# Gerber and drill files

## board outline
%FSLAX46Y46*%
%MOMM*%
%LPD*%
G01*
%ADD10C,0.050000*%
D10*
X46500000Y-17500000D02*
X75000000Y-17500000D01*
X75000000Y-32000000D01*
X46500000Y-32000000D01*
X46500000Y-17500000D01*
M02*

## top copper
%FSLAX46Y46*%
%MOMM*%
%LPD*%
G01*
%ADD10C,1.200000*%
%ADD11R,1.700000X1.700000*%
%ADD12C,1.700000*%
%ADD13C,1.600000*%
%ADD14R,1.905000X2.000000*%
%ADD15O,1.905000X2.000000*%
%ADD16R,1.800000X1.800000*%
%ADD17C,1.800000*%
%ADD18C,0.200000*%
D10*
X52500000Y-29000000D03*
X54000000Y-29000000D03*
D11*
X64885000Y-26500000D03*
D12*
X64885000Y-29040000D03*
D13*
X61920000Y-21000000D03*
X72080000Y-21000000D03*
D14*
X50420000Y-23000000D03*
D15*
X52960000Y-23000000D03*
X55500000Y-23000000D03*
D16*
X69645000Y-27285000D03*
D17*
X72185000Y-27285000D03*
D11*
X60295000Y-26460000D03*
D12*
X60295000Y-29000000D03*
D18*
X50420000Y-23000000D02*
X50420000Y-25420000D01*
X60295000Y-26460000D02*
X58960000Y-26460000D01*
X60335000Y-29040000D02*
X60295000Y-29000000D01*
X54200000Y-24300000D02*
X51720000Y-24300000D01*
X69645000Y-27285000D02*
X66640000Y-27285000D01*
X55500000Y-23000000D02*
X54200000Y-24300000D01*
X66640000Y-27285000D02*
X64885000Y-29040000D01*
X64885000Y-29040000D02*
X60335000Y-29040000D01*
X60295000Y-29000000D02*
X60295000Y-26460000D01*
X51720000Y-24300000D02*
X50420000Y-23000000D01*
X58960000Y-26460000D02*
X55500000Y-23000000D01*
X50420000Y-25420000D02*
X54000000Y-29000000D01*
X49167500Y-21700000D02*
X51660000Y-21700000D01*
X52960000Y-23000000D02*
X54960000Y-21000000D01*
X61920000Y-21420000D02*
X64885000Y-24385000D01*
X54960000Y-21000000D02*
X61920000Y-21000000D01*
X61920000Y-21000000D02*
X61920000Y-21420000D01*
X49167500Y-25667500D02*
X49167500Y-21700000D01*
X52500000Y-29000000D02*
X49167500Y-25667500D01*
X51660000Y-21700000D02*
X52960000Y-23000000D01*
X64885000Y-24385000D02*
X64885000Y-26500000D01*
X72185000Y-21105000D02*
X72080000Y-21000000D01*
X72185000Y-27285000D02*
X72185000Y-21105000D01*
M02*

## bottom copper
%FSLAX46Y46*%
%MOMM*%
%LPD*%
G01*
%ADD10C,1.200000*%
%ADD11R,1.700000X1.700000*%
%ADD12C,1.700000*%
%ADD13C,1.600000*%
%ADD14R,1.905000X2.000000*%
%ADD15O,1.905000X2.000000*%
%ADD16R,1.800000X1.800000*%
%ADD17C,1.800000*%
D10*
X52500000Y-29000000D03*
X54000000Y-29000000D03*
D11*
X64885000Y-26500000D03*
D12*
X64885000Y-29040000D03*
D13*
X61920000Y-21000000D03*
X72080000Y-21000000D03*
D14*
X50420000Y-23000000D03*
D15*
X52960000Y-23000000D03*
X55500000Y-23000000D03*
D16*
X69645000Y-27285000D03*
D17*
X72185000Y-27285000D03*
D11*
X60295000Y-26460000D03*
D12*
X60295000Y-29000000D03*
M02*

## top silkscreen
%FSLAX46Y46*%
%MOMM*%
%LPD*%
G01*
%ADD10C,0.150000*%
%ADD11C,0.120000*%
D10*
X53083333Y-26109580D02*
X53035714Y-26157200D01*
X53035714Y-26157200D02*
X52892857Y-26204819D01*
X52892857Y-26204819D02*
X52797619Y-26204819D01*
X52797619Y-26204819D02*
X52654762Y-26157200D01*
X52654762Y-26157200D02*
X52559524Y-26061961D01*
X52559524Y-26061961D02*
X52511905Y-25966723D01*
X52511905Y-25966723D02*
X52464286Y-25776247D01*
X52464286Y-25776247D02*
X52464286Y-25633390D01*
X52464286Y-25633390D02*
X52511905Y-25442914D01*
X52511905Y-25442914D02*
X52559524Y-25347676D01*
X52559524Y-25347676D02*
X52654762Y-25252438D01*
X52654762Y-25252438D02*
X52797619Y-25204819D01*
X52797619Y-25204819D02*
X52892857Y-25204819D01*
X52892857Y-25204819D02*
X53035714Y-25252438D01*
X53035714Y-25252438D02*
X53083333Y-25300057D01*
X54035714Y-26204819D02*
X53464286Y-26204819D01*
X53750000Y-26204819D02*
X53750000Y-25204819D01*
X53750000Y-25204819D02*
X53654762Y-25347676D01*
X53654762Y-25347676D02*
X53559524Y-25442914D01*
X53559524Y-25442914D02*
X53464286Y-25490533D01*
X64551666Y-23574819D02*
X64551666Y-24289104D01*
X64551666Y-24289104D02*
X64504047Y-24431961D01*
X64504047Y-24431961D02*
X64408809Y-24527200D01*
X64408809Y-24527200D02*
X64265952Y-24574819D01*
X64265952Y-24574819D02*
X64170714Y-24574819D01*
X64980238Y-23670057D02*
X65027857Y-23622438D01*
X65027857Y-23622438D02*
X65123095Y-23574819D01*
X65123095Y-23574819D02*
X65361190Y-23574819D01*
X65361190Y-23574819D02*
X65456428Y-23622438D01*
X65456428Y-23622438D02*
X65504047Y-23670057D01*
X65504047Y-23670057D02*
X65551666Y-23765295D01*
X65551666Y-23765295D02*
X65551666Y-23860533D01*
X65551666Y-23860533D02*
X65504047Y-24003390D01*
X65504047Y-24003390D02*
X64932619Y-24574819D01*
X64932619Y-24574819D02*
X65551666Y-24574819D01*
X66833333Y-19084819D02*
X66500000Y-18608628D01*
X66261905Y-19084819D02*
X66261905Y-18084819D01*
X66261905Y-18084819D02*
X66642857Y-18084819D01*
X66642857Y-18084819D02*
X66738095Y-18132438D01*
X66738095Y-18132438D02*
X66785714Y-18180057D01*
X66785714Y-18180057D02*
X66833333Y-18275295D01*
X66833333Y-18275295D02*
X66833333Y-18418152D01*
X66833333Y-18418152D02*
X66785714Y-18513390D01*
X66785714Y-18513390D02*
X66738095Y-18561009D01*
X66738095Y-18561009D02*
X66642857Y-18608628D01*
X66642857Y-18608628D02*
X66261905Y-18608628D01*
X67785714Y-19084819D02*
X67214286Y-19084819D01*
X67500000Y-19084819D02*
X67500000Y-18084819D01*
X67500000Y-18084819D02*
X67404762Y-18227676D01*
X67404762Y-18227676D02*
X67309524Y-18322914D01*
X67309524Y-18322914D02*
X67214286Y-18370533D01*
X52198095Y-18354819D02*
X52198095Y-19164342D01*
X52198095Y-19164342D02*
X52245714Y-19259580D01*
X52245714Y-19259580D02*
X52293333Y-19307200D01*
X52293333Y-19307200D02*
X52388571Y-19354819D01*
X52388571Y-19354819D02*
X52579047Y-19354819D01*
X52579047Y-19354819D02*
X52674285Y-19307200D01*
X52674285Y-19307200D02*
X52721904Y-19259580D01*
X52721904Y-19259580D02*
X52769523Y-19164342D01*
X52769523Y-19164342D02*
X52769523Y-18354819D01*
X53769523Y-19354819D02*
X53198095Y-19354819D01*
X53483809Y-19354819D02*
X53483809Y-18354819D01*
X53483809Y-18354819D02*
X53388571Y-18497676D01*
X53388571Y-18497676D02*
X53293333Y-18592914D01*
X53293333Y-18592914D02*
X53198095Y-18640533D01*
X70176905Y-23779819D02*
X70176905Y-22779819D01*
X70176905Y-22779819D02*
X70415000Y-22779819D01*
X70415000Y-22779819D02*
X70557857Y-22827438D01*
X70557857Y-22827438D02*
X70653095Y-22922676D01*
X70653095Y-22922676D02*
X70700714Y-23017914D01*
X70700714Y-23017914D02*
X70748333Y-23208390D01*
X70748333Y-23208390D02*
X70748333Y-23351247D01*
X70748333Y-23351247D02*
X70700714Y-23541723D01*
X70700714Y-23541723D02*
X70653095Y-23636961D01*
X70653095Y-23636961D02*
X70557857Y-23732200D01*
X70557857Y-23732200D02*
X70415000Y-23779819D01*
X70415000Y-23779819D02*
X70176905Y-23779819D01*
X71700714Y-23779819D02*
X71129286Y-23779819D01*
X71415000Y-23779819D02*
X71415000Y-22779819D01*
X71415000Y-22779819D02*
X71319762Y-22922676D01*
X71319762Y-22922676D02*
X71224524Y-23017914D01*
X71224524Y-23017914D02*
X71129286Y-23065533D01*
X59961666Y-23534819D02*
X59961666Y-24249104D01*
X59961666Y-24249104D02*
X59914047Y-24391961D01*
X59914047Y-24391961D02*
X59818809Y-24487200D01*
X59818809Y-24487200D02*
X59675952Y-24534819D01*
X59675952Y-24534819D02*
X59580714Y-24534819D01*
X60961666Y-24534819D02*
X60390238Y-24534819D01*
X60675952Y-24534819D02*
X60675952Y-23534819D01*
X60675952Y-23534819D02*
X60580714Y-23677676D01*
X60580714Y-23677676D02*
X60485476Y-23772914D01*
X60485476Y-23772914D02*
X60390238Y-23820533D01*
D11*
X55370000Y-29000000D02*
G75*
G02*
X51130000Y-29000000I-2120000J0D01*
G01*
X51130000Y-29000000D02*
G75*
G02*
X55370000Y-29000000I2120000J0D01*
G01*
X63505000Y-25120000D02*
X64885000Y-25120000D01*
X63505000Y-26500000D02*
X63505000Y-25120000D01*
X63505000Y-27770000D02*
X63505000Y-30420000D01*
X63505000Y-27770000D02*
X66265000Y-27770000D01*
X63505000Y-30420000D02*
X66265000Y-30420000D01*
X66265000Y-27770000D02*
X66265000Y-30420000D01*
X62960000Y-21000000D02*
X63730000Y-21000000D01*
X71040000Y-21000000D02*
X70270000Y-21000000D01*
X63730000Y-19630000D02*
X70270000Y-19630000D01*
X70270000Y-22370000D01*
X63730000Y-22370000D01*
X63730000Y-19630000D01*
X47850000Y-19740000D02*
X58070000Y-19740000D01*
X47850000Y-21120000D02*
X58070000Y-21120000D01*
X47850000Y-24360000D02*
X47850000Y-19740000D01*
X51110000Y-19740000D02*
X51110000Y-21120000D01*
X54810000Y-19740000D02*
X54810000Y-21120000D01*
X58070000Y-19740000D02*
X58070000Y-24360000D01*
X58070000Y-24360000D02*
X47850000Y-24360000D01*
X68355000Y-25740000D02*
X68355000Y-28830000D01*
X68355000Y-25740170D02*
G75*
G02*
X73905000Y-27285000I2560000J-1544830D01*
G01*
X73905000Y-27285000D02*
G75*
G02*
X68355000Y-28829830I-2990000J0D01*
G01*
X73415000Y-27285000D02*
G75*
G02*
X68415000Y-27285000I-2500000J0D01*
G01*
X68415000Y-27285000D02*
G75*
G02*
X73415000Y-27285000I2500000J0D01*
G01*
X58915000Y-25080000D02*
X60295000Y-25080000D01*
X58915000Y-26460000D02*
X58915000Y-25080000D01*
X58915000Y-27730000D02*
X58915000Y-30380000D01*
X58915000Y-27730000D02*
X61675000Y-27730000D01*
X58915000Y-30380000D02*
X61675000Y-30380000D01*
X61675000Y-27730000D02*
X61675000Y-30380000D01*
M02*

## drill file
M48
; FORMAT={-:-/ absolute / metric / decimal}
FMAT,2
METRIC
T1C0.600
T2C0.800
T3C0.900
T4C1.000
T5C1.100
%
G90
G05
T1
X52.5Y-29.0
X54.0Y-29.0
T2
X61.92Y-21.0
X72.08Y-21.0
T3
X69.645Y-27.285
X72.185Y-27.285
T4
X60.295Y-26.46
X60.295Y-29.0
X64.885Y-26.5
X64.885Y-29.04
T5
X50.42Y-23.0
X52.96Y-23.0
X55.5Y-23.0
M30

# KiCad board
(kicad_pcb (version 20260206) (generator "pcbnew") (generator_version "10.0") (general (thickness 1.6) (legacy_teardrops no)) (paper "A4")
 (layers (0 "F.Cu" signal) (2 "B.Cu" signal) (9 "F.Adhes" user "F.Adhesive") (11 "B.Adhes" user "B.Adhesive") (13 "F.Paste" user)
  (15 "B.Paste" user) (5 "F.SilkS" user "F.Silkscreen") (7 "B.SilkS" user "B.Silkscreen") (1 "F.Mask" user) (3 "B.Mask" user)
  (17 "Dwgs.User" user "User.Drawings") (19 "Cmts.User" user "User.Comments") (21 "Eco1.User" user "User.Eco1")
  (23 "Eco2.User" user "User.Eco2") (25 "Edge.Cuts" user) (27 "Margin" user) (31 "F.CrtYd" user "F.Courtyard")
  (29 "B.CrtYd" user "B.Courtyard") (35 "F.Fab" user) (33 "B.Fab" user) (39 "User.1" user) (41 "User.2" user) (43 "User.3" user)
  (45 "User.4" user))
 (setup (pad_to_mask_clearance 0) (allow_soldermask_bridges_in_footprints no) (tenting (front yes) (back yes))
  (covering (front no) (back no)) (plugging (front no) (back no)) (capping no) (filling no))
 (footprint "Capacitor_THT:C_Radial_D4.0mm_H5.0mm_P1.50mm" (layer "F.Cu") (at 52.5 29)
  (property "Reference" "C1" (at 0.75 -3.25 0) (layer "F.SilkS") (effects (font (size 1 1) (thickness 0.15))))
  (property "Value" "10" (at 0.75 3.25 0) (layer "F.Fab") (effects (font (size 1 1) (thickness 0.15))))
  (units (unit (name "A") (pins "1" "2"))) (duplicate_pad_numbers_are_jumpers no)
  (fp_circle (center 0.75 0) (end 2.87 0) (stroke (width 0.12) (type solid)) (fill no) (layer "F.SilkS"))
  (pad "1" thru_hole circle (at 0 0) (size 1.2 1.2) (drill 0.6) (layers "*.Cu" "*.Mask") (remove_unused_layers no) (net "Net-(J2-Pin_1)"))
  (pad "2" thru_hole circle (at 1.5 0) (size 1.2 1.2) (drill 0.6) (layers "*.Cu" "*.Mask") (remove_unused_layers no) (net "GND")))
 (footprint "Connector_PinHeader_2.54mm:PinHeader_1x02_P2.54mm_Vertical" (layer "F.Cu") (at 64.885 26.5)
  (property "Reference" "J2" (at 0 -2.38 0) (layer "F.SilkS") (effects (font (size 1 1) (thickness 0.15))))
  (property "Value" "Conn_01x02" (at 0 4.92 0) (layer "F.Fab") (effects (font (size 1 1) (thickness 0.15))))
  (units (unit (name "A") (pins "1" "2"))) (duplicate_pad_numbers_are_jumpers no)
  (fp_line (start -1.38 -1.38) (end 0 -1.38) (stroke (width 0.12) (type solid)) (layer "F.SilkS"))
  (fp_line (start -1.38 0) (end -1.38 -1.38) (stroke (width 0.12) (type solid)) (layer "F.SilkS"))
  (fp_line (start -1.38 1.27) (end -1.38 3.92) (stroke (width 0.12) (type solid)) (layer "F.SilkS"))
  (fp_line (start -1.38 1.27) (end 1.38 1.27) (stroke (width 0.12) (type solid)) (layer "F.SilkS"))
  (fp_line (start -1.38 3.92) (end 1.38 3.92) (stroke (width 0.12) (type solid)) (layer "F.SilkS"))
  (fp_line (start 1.38 1.27) (end 1.38 3.92) (stroke (width 0.12) (type solid)) (layer "F.SilkS"))
  (pad "1" thru_hole rect (at 0 0) (size 1.7 1.7) (drill 1) (layers "*.Cu" "*.Mask") (remove_unused_layers no) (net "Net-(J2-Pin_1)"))
  (pad "2" thru_hole circle (at 0 2.54) (size 1.7 1.7) (drill 1) (layers "*.Cu" "*.Mask") (remove_unused_layers no) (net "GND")))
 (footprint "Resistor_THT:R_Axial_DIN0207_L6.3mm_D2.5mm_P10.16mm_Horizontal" (layer "F.Cu") (at 61.92 21)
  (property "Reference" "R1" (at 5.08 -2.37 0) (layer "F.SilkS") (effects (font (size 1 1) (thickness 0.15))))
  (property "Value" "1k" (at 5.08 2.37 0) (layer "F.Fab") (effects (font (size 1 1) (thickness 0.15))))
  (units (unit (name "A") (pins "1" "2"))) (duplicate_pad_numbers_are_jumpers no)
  (fp_line (start 1.04 0) (end 1.81 0) (stroke (width 0.12) (type solid)) (layer "F.SilkS"))
  (fp_line (start 9.12 0) (end 8.35 0) (stroke (width 0.12) (type solid)) (layer "F.SilkS"))
  (fp_rect (start 1.81 -1.37) (end 8.35 1.37) (stroke (width 0.12) (type solid)) (fill no) (layer "F.SilkS"))
  (pad "1" thru_hole circle (at 0 0) (size 1.6 1.6) (drill 0.8) (layers "*.Cu" "*.Mask") (remove_unused_layers no) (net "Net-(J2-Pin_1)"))
  (pad "2" thru_hole circle (at 10.16 0) (size 1.6 1.6) (drill 0.8) (layers "*.Cu" "*.Mask") (remove_unused_layers no) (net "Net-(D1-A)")))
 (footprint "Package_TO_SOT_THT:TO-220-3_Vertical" (layer "F.Cu") (at 50.42 23)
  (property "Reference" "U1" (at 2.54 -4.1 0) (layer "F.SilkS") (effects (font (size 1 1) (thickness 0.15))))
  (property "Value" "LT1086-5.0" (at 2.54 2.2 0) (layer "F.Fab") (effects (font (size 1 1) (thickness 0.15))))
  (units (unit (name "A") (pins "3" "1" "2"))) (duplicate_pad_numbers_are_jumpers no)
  (fp_line (start -2.57 -3.26) (end 7.65 -3.26) (stroke (width 0.12) (type solid)) (layer "F.SilkS"))
  (fp_line (start -2.57 -1.88) (end 7.65 -1.88) (stroke (width 0.12) (type solid)) (layer "F.SilkS"))
  (fp_line (start -2.57 1.36) (end -2.57 -3.26) (stroke (width 0.12) (type solid)) (layer "F.SilkS"))
  (fp_line (start 0.69 -3.26) (end 0.69 -1.88) (stroke (width 0.12) (type solid)) (layer "F.SilkS"))
  (fp_line (start 4.39 -3.26) (end 4.39 -1.88) (stroke (width 0.12) (type solid)) (layer "F.SilkS"))
  (fp_line (start 7.65 -3.26) (end 7.65 1.36) (stroke (width 0.12) (type solid)) (layer "F.SilkS"))
  (fp_line (start 7.65 1.36) (end -2.57 1.36) (stroke (width 0.12) (type solid)) (layer "F.SilkS"))
  (pad "1" thru_hole rect (at 0 0) (size 1.905 2) (drill 1.1) (layers "*.Cu" "*.Mask") (remove_unused_layers no) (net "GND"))
  (pad "2" thru_hole oval (at 2.54 0) (size 1.905 2) (drill 1.1) (layers "*.Cu" "*.Mask") (remove_unused_layers no) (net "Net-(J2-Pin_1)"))
  (pad "3" thru_hole oval (at 5.08 0) (size 1.905 2) (drill 1.1) (layers "*.Cu" "*.Mask") (remove_unused_layers no) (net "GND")))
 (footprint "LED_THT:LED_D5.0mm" (layer "F.Cu") (at 69.645 27.285)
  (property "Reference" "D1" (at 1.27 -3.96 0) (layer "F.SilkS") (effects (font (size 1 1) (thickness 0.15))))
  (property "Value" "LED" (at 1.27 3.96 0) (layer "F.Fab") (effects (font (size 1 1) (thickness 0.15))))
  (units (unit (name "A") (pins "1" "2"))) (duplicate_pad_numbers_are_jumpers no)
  (fp_line (start -1.29 -1.545) (end -1.29 1.545) (stroke (width 0.12) (type solid)) (layer "F.SilkS"))
  (fp_arc (start -1.29 -1.54483) (mid 2.071779 -2.880495) (end 4.26 0) (stroke (width 0.12) (type solid)) (layer "F.SilkS"))
  (fp_arc (start 4.26 0) (mid 2.071779 2.880495) (end -1.29 1.54483) (stroke (width 0.12) (type solid)) (layer "F.SilkS"))
  (fp_circle (center 1.27 0) (end 3.77 0) (stroke (width 0.12) (type solid)) (fill no) (layer "F.SilkS"))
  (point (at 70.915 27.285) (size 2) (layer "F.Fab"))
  (pad "1" thru_hole rect (at 0 0) (size 1.8 1.8) (drill 0.9) (layers "*.Cu" "*.Mask") (remove_unused_layers no) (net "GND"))
  (pad "2" thru_hole circle (at 2.54 0) (size 1.8 1.8) (drill 0.9) (layers "*.Cu" "*.Mask") (remove_unused_layers no) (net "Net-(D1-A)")))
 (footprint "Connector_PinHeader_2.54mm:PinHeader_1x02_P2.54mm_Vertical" (layer "F.Cu") (at 60.295 26.46)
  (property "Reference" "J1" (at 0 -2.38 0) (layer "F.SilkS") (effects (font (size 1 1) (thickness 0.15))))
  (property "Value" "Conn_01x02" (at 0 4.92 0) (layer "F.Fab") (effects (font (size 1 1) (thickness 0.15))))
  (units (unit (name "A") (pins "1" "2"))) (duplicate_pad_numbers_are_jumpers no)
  (fp_line (start -1.38 -1.38) (end 0 -1.38) (stroke (width 0.12) (type solid)) (layer "F.SilkS"))
  (fp_line (start -1.38 0) (end -1.38 -1.38) (stroke (width 0.12) (type solid)) (layer "F.SilkS"))
  (fp_line (start -1.38 1.27) (end -1.38 3.92) (stroke (width 0.12) (type solid)) (layer "F.SilkS"))
  (fp_line (start -1.38 1.27) (end 1.38 1.27) (stroke (width 0.12) (type solid)) (layer "F.SilkS"))
  (fp_line (start -1.38 3.92) (end 1.38 3.92) (stroke (width 0.12) (type solid)) (layer "F.SilkS"))
  (fp_line (start 1.38 1.27) (end 1.38 3.92) (stroke (width 0.12) (type solid)) (layer "F.SilkS"))
  (pad "1" thru_hole rect (at 0 0) (size 1.7 1.7) (drill 1) (layers "*.Cu" "*.Mask") (remove_unused_layers no) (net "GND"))
  (pad "2" thru_hole circle (at 0 2.54) (size 1.7 1.7) (drill 1) (layers "*.Cu" "*.Mask") (remove_unused_layers no) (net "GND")))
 (gr_rect (start 46.5 17.5) (end 75 32) (stroke (width 0.05) (type default)) (fill no) (layer "Edge.Cuts"))
 (segment (start 50.42 23) (end 50.42 25.42) (width 0.2) (layer "F.Cu") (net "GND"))
 (segment (start 60.295 26.46) (end 58.96 26.46) (width 0.2) (layer "F.Cu") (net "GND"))
 (segment (start 60.335 29.04) (end 60.295 29) (width 0.2) (layer "F.Cu") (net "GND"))
 (segment (start 54.2 24.3) (end 51.72 24.3) (width 0.2) (layer "F.Cu") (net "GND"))
 (segment (start 69.645 27.285) (end 66.64 27.285) (width 0.2) (layer "F.Cu") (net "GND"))
 (segment (start 55.5 23) (end 54.2 24.3) (width 0.2) (layer "F.Cu") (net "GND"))
 (segment (start 66.64 27.285) (end 64.885 29.04) (width 0.2) (layer "F.Cu") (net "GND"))
 (segment (start 64.885 29.04) (end 60.335 29.04) (width 0.2) (layer "F.Cu") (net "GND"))
 (segment (start 60.295 29) (end 60.295 26.46) (width 0.2) (layer "F.Cu") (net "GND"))
 (segment (start 51.72 24.3) (end 50.42 23) (width 0.2) (layer "F.Cu") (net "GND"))
 (segment (start 58.96 26.46) (end 55.5 23) (width 0.2) (layer "F.Cu") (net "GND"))
 (segment (start 50.42 25.42) (end 54 29) (width 0.2) (layer "F.Cu") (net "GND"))
 (segment (start 49.1675 21.7) (end 51.66 21.7) (width 0.2) (layer "F.Cu") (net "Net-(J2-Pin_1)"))
 (segment (start 52.96 23) (end 54.96 21) (width 0.2) (layer "F.Cu") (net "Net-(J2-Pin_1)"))
 (segment (start 61.92 21.42) (end 64.885 24.385) (width 0.2) (layer "F.Cu") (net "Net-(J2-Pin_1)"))
 (segment (start 54.96 21) (end 61.92 21) (width 0.2) (layer "F.Cu") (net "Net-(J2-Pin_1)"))
 (segment (start 61.92 21) (end 61.92 21.42) (width 0.2) (layer "F.Cu") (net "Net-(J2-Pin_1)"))
 (segment (start 49.1675 25.6675) (end 49.1675 21.7) (width 0.2) (layer "F.Cu") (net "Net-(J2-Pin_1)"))
 (segment (start 52.5 29) (end 49.1675 25.6675) (width 0.2) (layer "F.Cu") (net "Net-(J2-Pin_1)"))
 (segment (start 51.66 21.7) (end 52.96 23) (width 0.2) (layer "F.Cu") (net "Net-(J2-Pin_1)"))
 (segment (start 64.885 24.385) (end 64.885 26.5) (width 0.2) (layer "F.Cu") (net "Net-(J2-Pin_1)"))
 (segment (start 72.185 21.105) (end 72.08 21) (width 0.2) (layer "F.Cu") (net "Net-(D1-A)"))
 (segment (start 72.185 27.285) (end 72.185 21.105) (width 0.2) (layer "F.Cu") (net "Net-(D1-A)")))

